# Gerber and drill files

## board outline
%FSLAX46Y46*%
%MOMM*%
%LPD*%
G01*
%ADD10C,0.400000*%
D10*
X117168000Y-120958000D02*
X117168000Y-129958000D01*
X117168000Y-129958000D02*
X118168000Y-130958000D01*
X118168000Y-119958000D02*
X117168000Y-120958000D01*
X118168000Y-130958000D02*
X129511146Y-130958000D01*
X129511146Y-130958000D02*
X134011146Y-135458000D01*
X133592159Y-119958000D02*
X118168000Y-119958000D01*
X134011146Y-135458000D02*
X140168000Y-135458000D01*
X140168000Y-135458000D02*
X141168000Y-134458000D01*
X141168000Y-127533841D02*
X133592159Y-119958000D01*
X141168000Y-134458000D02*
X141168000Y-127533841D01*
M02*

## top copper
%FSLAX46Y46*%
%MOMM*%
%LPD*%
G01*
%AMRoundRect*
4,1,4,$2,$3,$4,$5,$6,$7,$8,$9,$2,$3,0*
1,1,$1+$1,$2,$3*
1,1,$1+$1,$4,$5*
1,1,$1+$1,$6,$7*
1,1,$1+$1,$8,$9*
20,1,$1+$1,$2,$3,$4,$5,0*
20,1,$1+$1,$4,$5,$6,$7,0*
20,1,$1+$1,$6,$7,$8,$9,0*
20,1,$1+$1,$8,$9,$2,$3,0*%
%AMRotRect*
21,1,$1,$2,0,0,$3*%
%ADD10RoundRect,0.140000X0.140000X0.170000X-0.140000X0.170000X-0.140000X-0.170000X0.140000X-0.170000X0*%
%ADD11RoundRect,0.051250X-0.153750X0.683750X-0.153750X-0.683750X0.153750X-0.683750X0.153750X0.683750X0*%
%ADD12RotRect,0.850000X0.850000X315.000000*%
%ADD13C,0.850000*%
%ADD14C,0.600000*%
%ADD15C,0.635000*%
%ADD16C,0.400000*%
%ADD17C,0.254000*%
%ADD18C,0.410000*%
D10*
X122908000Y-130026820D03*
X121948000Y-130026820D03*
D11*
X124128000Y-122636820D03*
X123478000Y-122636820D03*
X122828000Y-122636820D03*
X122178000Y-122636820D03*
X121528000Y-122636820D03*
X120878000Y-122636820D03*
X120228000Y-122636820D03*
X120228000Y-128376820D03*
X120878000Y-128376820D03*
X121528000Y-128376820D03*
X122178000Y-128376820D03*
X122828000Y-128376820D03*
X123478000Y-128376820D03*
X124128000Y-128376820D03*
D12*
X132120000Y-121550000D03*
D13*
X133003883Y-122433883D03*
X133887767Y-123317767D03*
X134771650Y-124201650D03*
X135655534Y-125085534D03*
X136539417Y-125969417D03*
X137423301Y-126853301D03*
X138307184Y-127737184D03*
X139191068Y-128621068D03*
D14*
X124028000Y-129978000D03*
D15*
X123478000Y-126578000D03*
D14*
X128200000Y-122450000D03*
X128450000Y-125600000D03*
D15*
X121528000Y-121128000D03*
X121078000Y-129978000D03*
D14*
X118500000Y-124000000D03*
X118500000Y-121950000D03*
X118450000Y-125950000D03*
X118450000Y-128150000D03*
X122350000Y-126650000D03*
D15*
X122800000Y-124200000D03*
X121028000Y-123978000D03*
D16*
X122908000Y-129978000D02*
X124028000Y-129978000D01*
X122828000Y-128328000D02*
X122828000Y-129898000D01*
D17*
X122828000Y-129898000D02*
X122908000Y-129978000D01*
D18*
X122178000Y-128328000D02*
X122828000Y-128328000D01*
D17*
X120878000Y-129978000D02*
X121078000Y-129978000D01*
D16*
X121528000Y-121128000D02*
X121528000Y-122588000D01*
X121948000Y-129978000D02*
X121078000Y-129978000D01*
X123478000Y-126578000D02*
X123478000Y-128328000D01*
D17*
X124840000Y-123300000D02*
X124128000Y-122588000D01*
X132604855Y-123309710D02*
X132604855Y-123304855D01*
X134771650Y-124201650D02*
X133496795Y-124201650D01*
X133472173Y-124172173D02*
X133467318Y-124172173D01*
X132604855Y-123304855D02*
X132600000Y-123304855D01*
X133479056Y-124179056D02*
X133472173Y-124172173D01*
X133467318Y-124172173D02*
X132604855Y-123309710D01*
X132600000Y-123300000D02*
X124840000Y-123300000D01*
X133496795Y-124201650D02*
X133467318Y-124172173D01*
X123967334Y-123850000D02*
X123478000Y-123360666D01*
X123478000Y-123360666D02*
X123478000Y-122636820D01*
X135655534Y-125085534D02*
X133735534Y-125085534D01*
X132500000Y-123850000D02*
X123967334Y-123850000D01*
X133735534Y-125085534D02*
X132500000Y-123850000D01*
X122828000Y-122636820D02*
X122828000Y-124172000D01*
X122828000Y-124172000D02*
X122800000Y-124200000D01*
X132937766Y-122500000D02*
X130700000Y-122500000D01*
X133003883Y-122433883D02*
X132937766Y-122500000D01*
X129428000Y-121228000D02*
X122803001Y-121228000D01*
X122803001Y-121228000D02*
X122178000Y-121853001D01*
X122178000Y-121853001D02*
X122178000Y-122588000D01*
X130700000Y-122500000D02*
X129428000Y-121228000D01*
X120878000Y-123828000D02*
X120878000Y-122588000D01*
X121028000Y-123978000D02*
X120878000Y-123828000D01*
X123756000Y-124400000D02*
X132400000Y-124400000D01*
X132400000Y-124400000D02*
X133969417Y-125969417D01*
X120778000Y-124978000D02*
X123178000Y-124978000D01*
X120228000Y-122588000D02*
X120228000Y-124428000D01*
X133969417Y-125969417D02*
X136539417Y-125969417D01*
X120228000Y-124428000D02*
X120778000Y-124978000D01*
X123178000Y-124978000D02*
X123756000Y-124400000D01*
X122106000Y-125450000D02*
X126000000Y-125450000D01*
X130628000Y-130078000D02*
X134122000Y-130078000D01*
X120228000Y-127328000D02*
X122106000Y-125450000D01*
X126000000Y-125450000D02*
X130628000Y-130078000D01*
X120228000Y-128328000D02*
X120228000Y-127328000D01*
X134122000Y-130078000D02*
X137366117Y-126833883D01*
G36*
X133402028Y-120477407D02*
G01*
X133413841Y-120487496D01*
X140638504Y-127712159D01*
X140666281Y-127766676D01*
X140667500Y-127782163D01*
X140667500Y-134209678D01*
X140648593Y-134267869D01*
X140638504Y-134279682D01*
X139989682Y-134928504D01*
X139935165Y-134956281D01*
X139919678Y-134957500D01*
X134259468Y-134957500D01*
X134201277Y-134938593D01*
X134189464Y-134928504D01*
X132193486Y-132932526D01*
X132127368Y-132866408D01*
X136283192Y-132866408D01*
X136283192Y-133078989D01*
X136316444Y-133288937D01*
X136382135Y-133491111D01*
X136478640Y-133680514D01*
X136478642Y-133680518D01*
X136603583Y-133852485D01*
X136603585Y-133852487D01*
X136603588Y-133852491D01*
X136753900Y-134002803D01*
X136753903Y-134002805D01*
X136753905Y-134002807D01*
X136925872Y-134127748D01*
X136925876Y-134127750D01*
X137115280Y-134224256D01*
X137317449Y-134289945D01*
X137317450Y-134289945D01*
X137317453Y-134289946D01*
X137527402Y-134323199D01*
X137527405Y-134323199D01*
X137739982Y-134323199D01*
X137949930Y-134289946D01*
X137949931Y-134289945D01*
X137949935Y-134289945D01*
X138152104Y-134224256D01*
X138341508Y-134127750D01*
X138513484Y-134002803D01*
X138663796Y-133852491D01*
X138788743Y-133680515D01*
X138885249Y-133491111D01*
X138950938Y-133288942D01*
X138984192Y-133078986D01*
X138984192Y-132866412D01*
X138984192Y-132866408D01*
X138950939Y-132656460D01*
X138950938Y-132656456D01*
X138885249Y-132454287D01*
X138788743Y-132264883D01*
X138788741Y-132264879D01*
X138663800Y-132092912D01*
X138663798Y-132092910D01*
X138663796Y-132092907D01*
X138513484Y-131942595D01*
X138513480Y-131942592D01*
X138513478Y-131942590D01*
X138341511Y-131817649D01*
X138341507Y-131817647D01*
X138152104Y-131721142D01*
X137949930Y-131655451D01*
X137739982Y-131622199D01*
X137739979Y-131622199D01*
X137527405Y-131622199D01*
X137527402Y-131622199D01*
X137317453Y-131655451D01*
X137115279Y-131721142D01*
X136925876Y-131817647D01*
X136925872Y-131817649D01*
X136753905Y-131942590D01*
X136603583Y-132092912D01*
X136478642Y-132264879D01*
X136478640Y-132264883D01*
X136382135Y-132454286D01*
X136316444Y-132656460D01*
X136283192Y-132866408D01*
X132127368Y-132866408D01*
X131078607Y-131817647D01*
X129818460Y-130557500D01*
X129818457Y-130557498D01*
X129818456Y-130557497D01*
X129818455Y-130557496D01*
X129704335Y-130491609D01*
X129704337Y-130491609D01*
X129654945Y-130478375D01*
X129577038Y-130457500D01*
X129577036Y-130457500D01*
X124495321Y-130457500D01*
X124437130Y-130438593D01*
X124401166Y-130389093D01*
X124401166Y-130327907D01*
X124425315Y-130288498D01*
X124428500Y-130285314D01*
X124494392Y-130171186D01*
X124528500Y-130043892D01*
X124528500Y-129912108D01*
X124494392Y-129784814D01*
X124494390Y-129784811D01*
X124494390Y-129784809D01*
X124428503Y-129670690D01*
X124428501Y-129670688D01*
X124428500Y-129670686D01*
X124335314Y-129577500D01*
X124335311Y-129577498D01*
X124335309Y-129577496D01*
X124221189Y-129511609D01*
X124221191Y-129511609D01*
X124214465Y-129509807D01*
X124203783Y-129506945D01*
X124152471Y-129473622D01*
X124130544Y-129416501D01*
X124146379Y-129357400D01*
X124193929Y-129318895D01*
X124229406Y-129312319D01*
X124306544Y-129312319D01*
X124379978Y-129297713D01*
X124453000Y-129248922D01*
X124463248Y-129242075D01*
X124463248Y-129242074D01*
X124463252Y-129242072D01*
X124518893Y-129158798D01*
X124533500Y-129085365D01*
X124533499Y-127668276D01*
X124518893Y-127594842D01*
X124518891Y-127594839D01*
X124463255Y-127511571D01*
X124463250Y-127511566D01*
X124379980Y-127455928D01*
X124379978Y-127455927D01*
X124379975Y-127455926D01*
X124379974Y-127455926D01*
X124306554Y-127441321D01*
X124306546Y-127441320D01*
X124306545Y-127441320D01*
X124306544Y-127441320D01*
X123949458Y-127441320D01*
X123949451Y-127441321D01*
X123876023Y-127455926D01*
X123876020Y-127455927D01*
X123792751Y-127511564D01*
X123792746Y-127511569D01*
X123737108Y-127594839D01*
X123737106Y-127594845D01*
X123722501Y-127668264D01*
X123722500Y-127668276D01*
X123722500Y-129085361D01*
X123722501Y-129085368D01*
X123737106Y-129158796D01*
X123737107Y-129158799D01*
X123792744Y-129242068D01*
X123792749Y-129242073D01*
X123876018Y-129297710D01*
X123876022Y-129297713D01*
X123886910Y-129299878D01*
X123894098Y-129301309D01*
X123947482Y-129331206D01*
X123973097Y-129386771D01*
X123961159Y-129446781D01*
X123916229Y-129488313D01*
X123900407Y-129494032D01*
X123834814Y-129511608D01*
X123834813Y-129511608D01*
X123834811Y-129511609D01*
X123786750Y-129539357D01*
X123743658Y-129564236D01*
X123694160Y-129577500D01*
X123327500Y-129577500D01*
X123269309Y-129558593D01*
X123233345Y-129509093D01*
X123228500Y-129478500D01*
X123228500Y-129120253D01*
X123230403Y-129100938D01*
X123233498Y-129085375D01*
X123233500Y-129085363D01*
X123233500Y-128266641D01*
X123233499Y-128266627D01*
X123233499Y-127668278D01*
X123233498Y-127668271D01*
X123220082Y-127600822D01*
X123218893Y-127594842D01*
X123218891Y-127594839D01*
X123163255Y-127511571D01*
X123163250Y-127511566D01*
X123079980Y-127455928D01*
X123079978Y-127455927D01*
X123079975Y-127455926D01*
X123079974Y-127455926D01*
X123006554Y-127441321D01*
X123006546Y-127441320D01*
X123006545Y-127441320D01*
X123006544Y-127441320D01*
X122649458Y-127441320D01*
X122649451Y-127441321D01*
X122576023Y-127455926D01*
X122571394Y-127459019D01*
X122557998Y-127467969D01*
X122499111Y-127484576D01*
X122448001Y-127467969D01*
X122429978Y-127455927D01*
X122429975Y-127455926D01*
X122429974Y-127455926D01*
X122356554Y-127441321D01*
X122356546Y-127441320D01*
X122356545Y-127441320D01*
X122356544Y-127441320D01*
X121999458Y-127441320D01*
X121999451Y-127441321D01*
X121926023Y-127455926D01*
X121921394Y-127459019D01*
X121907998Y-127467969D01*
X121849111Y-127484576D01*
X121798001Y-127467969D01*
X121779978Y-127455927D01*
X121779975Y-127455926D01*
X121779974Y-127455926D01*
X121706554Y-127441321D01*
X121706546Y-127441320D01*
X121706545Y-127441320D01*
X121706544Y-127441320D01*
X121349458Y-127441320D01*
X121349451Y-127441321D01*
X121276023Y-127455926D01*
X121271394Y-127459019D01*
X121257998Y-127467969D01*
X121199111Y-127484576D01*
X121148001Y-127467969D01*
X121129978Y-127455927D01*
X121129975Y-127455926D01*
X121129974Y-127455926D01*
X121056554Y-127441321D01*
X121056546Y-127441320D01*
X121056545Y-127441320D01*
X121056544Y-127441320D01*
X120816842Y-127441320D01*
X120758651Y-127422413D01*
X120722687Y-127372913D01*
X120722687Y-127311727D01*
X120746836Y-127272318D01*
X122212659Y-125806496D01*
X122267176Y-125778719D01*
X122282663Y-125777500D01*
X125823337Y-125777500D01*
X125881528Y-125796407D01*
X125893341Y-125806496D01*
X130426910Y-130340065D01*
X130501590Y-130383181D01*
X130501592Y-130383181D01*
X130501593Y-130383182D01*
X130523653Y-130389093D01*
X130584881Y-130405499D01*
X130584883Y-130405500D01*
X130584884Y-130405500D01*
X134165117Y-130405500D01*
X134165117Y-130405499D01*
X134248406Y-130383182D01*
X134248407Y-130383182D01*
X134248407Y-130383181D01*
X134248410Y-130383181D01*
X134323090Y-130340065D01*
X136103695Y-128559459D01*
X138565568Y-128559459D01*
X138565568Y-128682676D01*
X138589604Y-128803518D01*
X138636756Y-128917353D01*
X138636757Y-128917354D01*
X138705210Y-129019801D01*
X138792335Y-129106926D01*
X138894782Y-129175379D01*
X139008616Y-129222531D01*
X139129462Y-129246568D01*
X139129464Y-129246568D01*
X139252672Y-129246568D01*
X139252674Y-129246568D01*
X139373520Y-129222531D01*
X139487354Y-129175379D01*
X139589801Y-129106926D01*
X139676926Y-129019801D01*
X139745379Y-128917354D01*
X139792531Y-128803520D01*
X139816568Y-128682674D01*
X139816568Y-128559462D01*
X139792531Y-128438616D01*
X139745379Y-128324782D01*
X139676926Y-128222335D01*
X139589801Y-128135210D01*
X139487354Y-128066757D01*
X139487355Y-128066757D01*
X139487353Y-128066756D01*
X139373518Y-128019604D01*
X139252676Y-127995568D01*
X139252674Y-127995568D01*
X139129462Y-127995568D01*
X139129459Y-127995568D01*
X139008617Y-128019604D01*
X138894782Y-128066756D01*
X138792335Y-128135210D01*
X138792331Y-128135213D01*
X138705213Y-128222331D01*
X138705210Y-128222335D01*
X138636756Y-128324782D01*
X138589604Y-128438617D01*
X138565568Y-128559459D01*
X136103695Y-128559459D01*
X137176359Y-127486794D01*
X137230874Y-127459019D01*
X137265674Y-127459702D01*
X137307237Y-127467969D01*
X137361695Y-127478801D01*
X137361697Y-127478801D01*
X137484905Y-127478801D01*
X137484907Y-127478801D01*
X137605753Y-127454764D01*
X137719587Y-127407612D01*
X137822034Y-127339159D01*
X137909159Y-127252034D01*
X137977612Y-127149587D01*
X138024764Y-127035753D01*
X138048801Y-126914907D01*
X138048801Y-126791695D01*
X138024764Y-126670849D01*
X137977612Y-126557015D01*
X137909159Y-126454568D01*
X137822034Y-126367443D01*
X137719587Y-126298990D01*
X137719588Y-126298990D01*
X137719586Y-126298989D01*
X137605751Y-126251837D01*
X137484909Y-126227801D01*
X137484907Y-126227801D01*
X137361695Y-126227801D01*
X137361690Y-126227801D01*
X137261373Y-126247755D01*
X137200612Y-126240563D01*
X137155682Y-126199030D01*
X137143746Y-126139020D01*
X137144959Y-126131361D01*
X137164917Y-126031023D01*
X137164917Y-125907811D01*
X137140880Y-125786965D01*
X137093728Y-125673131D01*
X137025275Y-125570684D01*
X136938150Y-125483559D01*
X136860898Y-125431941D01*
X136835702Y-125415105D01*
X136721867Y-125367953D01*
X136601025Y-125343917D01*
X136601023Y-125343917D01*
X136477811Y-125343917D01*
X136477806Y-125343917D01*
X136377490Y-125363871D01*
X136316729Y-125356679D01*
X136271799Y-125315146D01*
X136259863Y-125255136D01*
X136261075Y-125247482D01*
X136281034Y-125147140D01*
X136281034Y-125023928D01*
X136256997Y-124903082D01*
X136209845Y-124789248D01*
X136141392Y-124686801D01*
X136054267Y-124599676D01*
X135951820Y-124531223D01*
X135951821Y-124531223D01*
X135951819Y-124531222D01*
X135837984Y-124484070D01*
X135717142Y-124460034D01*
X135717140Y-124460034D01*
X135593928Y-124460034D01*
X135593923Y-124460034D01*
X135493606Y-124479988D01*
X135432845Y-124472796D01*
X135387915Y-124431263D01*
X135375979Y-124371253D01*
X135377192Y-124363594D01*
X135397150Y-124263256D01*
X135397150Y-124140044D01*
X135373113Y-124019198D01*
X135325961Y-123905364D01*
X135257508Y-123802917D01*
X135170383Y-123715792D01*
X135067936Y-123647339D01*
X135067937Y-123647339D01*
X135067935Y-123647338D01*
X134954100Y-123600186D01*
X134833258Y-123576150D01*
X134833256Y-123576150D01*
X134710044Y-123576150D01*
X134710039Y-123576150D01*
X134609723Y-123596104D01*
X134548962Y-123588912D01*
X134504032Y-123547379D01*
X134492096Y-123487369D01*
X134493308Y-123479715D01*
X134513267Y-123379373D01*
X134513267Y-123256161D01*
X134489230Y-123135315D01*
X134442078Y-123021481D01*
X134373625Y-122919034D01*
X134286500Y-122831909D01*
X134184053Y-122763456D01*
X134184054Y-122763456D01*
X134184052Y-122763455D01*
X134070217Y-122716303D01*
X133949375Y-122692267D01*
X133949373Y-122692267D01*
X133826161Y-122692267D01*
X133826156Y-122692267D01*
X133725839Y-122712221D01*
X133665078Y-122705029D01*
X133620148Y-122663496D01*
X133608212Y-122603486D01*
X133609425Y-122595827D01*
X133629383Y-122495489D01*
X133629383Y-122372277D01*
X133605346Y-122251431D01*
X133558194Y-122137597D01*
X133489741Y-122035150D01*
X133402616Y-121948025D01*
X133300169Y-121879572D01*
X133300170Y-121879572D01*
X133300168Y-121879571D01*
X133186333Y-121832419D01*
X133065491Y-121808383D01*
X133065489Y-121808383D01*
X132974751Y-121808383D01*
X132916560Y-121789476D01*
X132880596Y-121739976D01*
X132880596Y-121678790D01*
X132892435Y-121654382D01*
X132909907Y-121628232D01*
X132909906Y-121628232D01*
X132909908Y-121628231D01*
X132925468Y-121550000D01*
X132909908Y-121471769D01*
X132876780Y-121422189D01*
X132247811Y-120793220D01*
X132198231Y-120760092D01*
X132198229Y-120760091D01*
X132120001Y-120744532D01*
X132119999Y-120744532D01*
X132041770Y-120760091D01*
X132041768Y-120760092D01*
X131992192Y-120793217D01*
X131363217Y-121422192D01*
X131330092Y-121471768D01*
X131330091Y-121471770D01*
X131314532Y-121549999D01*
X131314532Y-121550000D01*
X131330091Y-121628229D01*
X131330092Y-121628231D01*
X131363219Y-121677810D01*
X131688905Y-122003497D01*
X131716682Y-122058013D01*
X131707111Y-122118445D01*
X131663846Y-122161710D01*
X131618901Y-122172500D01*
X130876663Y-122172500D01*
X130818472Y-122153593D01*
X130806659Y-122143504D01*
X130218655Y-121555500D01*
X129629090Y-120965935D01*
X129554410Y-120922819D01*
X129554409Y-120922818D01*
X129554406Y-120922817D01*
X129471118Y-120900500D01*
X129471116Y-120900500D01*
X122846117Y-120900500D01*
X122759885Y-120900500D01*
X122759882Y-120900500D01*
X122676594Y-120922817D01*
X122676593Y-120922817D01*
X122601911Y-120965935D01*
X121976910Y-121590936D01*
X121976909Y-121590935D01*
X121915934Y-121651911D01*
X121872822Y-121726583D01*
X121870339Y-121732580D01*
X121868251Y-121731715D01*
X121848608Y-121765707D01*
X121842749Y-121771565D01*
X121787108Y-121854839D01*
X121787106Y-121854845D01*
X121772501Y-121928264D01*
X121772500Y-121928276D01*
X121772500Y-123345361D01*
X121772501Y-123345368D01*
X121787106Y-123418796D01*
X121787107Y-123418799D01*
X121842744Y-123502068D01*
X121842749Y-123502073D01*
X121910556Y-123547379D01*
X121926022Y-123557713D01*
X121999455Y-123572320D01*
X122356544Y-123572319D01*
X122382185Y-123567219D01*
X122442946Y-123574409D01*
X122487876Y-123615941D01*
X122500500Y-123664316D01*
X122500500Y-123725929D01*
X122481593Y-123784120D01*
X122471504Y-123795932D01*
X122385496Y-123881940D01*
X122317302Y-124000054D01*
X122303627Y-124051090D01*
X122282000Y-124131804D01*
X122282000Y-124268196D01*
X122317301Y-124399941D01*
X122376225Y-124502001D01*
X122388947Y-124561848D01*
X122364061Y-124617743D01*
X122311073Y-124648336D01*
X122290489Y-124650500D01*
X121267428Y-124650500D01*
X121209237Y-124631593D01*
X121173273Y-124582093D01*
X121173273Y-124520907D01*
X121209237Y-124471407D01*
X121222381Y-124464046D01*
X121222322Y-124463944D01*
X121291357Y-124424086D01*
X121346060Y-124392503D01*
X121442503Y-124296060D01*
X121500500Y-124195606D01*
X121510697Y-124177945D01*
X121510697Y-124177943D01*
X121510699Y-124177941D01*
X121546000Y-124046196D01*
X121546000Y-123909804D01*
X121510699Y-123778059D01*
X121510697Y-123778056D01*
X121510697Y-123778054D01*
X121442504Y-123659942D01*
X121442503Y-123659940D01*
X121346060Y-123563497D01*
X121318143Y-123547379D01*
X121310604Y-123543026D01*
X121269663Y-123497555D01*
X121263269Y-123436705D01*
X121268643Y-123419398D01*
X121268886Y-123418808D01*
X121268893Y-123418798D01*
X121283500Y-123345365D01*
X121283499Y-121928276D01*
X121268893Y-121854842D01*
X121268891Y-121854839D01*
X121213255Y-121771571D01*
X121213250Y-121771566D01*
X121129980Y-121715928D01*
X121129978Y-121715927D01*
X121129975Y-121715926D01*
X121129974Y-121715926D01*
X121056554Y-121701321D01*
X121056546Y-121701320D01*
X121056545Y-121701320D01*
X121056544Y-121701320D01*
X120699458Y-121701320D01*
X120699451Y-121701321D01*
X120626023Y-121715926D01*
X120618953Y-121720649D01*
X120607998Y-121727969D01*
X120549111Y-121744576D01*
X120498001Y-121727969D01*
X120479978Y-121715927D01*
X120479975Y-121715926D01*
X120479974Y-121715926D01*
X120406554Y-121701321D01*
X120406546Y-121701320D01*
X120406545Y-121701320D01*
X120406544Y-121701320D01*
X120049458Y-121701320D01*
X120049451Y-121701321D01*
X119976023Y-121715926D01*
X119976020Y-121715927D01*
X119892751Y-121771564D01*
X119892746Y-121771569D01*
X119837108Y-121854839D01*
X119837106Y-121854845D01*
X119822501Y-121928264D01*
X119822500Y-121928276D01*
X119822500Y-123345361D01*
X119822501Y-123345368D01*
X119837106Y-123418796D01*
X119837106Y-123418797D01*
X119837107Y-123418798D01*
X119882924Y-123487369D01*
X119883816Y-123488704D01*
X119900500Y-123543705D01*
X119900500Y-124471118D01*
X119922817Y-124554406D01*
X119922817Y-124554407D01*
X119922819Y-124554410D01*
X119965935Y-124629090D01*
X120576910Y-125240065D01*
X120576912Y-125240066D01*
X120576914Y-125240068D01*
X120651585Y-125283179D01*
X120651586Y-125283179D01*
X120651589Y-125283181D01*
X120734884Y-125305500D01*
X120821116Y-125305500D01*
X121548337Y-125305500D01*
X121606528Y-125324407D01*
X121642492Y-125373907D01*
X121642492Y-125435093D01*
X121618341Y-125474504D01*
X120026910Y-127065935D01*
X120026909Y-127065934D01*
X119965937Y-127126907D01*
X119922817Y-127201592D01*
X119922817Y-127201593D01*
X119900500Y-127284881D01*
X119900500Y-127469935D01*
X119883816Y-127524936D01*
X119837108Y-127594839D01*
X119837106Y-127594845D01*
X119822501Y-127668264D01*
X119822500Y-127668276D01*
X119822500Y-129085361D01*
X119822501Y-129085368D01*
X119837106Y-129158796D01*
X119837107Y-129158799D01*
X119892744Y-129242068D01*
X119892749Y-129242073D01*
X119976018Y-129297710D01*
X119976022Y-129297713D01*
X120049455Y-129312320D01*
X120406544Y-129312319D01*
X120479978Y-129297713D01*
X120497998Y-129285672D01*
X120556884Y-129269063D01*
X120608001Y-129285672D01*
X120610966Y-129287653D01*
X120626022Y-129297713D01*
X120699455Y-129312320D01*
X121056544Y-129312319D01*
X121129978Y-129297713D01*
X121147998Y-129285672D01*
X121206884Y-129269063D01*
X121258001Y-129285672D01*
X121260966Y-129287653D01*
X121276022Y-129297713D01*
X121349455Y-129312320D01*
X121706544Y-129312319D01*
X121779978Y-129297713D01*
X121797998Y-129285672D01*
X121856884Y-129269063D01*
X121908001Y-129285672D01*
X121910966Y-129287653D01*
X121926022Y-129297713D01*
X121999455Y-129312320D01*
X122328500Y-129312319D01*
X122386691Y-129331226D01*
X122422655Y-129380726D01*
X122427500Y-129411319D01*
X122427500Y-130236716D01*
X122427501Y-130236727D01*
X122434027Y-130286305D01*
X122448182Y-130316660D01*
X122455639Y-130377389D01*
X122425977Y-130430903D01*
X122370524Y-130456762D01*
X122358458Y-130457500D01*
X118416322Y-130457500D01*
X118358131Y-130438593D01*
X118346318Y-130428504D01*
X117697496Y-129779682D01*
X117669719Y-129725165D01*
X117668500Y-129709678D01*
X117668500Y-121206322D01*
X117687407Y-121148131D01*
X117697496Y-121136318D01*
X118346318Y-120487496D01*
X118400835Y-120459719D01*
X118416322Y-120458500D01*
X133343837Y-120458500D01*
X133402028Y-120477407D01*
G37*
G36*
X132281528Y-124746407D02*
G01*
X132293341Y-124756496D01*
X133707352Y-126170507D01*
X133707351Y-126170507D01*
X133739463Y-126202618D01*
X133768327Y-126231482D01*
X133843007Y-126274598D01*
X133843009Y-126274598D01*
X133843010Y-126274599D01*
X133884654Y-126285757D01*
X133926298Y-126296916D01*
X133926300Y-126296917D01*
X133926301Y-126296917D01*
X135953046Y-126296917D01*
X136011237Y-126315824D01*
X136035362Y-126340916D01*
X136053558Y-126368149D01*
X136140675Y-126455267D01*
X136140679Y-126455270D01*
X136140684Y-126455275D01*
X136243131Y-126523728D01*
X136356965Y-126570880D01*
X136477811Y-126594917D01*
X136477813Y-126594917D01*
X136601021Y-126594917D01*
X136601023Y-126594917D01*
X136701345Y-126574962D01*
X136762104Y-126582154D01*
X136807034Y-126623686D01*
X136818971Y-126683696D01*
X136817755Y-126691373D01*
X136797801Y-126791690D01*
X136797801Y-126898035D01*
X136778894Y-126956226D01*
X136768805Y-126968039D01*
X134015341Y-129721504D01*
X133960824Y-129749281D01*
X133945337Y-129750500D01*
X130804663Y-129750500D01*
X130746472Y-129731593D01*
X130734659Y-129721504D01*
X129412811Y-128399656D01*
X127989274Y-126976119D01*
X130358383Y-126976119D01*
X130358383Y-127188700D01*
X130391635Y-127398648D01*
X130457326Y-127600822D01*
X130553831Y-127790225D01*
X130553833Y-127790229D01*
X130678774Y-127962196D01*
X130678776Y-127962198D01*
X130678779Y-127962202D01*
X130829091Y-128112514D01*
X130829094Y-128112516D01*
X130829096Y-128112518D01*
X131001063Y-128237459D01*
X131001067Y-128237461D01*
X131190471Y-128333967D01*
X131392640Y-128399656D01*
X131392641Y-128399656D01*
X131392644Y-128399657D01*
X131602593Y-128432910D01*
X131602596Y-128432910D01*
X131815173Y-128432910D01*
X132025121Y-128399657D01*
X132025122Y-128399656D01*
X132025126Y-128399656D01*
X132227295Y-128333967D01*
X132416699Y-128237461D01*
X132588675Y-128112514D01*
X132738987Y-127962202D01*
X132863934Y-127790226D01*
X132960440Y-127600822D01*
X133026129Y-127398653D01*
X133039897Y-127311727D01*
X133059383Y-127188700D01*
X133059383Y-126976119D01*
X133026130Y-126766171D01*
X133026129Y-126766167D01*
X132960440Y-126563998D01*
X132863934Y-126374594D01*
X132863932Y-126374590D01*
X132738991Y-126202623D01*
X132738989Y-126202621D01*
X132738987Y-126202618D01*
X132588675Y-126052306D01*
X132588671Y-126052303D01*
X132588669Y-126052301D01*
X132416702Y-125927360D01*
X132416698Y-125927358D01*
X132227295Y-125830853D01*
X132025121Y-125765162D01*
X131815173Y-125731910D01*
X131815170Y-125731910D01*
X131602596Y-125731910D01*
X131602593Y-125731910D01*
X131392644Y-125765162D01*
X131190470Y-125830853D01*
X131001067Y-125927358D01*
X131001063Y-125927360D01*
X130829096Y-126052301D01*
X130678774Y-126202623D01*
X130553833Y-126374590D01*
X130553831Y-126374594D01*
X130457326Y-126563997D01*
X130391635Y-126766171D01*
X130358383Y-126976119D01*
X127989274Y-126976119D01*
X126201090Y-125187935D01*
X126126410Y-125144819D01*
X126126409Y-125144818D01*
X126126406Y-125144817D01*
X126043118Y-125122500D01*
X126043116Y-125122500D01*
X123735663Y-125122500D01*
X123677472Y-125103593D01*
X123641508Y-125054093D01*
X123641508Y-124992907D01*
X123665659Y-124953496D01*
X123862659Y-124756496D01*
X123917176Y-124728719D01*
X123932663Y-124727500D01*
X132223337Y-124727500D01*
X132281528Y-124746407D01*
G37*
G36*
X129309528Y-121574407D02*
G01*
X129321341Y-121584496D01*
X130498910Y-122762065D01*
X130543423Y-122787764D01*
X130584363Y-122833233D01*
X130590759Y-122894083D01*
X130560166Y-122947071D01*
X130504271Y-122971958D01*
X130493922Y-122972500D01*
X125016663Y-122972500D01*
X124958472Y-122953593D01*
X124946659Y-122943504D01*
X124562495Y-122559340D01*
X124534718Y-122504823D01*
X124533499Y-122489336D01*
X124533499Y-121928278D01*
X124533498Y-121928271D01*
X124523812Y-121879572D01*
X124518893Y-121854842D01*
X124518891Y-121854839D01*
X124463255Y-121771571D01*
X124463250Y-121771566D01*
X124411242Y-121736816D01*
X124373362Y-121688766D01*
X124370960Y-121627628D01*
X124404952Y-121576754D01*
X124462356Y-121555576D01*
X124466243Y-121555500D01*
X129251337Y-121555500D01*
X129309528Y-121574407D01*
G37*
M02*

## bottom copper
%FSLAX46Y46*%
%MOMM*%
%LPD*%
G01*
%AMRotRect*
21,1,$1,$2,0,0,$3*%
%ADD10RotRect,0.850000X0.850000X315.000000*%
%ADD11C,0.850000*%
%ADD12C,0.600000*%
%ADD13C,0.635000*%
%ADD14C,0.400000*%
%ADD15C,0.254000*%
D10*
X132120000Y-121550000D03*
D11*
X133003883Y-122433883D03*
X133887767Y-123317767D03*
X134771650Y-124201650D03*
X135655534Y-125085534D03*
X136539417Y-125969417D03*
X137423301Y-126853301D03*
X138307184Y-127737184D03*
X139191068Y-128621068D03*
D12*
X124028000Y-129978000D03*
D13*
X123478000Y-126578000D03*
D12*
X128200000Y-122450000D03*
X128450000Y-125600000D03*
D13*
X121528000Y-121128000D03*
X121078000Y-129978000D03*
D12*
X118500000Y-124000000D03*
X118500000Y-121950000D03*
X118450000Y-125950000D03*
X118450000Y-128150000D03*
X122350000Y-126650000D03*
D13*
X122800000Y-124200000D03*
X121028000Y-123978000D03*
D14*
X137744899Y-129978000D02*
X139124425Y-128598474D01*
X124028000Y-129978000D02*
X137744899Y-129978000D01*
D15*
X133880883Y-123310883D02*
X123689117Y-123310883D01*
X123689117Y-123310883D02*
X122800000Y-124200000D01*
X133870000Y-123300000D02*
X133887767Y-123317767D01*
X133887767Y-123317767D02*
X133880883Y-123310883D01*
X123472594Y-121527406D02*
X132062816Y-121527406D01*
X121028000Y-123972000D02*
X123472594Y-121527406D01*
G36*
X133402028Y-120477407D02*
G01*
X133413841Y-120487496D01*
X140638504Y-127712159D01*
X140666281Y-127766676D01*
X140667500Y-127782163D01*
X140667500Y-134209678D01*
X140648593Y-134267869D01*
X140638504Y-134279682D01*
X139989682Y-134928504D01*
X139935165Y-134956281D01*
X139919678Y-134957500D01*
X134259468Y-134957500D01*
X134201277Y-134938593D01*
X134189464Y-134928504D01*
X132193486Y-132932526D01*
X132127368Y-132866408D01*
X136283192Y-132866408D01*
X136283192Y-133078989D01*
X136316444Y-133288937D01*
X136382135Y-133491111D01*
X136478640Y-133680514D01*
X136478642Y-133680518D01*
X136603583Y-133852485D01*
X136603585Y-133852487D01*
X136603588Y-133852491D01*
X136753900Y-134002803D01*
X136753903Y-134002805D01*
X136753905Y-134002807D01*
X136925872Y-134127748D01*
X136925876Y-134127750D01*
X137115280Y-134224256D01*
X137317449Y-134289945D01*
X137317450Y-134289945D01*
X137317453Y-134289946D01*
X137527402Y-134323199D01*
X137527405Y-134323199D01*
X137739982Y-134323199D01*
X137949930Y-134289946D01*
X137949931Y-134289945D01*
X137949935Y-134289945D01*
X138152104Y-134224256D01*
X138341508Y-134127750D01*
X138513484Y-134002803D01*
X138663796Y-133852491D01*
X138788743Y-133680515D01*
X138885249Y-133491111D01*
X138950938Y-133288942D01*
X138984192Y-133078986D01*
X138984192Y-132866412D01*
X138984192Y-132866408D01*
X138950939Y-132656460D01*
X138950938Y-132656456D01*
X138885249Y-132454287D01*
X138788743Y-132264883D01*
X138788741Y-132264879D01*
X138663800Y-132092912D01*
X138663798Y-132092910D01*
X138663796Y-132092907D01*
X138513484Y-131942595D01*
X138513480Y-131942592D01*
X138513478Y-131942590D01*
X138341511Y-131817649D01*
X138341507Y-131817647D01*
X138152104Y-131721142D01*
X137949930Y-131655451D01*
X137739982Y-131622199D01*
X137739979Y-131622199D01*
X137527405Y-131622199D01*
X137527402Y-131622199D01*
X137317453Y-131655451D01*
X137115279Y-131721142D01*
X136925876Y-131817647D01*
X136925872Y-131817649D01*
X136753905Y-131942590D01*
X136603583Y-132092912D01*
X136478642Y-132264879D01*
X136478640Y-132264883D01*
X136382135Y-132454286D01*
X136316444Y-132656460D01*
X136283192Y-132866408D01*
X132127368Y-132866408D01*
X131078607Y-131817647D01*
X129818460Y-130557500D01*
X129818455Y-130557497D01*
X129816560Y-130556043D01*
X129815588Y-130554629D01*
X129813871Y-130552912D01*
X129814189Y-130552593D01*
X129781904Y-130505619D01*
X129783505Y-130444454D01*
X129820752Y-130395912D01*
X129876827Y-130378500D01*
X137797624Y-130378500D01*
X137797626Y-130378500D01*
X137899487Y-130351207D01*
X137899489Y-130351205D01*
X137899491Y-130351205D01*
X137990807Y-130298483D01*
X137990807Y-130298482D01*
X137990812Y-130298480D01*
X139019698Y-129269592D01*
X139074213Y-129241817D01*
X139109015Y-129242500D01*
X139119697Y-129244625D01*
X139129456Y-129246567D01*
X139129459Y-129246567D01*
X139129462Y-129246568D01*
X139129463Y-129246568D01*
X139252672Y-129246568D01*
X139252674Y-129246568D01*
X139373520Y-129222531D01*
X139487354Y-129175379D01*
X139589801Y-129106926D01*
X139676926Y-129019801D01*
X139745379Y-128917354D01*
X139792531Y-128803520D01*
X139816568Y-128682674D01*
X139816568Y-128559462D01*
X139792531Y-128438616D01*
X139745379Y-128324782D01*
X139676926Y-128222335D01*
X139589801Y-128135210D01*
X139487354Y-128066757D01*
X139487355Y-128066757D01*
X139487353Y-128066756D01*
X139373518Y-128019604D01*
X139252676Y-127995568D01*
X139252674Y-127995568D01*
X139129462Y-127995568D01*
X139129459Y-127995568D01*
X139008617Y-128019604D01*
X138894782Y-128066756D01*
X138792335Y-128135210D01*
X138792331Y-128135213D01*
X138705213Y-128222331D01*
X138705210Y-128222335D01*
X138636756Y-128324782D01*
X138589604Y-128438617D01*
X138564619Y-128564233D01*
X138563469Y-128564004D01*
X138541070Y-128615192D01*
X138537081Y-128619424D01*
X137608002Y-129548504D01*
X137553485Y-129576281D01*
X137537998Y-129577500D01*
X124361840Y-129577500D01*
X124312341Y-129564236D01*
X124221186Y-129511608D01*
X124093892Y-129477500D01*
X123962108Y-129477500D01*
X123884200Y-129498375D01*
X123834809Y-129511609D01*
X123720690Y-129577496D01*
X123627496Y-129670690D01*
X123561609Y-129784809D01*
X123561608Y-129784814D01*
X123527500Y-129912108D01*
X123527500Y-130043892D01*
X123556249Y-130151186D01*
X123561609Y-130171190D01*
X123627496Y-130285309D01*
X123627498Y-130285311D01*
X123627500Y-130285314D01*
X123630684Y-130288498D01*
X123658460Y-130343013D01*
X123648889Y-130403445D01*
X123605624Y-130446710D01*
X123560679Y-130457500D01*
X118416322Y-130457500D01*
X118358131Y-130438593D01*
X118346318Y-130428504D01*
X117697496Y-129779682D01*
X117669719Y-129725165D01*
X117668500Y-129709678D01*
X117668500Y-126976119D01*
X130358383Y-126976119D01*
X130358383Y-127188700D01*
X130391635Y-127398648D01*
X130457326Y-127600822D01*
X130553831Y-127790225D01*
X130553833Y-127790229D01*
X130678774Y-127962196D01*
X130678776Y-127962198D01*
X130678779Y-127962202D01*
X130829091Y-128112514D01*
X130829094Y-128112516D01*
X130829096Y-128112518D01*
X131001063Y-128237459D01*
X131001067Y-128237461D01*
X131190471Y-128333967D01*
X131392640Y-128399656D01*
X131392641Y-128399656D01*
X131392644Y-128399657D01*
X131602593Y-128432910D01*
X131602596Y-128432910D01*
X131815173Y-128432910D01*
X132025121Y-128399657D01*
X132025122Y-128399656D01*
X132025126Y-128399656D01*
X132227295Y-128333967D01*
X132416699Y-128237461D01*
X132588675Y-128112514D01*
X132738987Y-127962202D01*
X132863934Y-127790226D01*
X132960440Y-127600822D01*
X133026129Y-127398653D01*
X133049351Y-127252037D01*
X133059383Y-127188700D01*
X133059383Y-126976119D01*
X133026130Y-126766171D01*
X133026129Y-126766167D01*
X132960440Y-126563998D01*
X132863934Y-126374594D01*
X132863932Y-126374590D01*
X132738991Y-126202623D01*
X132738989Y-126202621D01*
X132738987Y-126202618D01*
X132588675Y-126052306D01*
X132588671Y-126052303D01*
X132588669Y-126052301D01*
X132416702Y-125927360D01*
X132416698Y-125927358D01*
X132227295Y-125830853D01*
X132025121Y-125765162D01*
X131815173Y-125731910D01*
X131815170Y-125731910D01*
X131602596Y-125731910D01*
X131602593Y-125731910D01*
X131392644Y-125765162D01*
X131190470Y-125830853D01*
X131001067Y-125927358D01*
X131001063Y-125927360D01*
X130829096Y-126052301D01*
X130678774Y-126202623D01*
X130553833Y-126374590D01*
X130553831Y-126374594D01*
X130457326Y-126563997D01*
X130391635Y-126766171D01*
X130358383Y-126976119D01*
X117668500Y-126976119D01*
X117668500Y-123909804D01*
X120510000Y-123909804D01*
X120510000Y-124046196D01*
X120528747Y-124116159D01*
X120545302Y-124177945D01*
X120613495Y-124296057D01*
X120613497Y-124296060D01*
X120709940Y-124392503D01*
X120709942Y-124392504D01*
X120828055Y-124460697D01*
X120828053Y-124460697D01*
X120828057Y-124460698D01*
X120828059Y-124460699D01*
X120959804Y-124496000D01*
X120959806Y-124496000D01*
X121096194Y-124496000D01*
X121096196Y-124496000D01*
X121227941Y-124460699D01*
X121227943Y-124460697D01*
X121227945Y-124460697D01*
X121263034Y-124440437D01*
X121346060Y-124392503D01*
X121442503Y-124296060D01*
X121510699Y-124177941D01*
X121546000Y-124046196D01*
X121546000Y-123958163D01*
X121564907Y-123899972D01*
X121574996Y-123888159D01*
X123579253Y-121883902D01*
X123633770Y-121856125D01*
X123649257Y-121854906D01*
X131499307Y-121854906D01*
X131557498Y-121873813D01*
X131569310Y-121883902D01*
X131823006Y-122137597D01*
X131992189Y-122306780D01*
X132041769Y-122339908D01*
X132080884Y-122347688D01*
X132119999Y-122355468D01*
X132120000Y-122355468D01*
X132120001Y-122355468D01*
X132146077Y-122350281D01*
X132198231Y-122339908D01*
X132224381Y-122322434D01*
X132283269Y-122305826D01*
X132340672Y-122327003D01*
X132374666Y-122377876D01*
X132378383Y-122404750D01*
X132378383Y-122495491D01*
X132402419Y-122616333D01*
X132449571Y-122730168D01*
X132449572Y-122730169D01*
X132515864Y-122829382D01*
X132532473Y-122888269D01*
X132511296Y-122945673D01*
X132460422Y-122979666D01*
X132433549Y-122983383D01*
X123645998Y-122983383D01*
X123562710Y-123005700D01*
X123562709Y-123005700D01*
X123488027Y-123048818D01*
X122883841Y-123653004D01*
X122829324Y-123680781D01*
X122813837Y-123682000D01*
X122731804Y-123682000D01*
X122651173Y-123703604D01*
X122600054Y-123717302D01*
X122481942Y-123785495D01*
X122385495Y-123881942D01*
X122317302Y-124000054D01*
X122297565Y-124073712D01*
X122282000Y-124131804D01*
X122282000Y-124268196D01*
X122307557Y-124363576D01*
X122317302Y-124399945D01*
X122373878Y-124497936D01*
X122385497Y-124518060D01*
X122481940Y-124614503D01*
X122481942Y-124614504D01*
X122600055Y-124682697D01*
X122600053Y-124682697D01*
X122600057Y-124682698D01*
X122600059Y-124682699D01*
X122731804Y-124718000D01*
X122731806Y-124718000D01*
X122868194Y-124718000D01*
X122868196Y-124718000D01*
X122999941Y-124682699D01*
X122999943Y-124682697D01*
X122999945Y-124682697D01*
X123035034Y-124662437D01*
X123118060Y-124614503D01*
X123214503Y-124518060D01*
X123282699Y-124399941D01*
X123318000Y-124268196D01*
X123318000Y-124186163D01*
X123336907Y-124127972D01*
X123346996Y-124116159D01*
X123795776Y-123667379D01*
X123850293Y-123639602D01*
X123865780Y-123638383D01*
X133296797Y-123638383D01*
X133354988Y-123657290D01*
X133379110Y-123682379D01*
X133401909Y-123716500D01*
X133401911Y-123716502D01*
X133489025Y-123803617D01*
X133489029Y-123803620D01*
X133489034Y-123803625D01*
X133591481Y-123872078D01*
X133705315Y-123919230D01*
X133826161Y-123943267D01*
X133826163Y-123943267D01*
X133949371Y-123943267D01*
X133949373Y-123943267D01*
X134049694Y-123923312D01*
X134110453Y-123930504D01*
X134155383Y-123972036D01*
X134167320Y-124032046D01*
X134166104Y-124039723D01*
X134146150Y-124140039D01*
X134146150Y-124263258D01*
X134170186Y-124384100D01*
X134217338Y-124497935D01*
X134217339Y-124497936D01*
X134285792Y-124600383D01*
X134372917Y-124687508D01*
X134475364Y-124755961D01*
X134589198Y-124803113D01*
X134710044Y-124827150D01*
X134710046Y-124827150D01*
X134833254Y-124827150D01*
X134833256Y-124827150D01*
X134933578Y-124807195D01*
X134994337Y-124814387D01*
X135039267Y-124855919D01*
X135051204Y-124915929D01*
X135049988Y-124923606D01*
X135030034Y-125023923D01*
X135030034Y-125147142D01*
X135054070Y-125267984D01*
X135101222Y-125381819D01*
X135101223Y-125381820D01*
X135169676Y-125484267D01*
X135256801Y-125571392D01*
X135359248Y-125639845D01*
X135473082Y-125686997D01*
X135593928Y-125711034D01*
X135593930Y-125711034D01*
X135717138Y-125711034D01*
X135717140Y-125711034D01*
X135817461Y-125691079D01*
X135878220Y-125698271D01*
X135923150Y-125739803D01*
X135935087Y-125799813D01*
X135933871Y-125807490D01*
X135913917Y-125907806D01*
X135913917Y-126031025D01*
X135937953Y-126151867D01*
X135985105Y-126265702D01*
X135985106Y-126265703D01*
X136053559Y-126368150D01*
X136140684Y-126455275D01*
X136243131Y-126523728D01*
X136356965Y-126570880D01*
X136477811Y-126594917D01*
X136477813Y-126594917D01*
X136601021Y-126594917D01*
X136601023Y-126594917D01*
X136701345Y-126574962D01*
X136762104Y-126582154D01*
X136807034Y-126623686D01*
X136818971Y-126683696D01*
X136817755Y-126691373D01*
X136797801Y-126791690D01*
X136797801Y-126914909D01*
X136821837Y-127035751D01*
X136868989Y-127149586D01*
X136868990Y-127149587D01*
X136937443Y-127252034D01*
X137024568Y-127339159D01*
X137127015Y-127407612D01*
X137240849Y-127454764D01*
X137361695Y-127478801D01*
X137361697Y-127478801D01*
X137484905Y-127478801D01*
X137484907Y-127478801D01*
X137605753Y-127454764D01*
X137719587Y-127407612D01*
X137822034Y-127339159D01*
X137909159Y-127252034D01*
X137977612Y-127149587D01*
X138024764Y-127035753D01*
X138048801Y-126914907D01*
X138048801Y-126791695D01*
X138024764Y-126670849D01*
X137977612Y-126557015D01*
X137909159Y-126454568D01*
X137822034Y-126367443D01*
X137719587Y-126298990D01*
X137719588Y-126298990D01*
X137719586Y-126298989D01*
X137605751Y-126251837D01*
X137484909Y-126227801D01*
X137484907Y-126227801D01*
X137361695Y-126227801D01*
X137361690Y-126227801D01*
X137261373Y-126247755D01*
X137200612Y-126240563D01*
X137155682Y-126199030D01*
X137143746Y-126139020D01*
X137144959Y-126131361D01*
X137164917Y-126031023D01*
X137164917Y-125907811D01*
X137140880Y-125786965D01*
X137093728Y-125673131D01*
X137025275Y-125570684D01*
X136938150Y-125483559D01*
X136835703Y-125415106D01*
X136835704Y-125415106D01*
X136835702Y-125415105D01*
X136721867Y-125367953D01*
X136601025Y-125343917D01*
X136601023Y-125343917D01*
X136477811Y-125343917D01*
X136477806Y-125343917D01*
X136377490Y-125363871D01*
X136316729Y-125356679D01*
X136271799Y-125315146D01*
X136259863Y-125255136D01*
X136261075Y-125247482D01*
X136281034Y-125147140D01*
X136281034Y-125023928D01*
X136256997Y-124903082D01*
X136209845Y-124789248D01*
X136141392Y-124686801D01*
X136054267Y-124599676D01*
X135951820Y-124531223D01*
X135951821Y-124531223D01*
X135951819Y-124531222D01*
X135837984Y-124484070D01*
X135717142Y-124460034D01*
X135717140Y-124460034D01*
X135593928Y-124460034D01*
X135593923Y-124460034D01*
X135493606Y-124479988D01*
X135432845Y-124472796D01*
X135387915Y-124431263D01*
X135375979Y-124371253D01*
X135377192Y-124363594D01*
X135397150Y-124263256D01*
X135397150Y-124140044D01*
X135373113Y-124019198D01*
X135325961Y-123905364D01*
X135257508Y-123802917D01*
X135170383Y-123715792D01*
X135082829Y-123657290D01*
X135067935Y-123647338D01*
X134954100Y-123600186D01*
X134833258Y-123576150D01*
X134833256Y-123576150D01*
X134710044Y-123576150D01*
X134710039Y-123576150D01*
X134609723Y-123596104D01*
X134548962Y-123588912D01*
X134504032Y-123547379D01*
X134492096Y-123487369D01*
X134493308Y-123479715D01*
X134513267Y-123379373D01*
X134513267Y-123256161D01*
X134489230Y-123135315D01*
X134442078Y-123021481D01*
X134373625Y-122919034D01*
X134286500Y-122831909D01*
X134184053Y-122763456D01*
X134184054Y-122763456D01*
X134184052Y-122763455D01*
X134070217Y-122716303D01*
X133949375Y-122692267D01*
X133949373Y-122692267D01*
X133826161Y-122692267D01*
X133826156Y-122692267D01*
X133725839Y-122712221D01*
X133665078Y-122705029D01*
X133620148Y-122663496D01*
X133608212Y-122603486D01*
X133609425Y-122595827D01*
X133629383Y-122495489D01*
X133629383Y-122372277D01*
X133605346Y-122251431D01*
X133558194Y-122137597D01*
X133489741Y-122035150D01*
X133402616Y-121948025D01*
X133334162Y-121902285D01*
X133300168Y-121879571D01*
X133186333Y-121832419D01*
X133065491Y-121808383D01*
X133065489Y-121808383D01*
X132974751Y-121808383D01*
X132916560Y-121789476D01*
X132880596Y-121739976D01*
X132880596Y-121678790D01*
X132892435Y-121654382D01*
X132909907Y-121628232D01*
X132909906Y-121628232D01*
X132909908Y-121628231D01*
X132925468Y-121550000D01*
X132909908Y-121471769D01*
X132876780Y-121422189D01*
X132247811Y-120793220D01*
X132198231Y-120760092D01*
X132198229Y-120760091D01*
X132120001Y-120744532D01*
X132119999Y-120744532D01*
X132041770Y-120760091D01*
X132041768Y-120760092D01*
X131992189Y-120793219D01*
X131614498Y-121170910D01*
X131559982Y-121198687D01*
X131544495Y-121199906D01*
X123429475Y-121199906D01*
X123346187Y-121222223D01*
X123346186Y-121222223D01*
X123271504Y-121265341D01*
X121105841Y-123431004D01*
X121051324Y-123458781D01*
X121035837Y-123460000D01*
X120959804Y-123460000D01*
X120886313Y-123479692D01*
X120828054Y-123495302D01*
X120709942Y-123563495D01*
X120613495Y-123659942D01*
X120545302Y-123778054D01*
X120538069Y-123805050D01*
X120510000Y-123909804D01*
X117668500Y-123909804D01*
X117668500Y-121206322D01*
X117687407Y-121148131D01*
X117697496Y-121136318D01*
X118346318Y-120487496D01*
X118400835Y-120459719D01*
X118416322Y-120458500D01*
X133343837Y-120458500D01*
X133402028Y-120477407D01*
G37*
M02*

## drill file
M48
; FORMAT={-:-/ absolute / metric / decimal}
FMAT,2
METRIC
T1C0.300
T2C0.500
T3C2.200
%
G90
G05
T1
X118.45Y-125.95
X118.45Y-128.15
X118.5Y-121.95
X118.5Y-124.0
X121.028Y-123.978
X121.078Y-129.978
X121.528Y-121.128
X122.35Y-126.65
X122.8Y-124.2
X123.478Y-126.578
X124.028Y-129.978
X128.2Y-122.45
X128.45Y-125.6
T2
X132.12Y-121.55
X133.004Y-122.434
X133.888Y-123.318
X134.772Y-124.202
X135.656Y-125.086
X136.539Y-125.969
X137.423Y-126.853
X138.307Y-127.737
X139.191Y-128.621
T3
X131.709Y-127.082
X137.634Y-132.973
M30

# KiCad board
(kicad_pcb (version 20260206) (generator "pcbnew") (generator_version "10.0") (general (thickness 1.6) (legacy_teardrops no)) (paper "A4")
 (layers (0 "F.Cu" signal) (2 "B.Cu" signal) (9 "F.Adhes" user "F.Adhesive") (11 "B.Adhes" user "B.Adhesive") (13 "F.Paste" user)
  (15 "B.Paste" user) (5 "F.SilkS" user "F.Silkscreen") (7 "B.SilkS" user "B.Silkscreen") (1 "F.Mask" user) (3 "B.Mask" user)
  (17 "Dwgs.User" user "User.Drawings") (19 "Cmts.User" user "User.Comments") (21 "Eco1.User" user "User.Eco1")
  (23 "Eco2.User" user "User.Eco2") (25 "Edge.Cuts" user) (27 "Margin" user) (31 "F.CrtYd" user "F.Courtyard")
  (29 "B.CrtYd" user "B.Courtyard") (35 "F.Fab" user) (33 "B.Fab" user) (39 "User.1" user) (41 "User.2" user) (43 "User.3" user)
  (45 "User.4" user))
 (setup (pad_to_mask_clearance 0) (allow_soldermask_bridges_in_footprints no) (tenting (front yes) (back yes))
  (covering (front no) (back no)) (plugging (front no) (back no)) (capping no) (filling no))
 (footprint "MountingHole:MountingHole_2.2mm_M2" (layer "F.Cu") (at 137.633692 132.972699)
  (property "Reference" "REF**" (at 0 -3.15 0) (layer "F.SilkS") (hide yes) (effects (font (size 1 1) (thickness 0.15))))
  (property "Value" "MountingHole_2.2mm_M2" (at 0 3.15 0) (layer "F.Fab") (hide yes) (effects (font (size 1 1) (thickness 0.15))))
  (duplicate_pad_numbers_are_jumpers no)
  (pad "" np_thru_hole circle (at 0 0) (size 2.2 2.2) (drill 2.2) (layers "*.Cu" "*.Mask")))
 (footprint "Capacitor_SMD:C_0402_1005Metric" (layer "F.Cu") (at 122.428 130.02682 180)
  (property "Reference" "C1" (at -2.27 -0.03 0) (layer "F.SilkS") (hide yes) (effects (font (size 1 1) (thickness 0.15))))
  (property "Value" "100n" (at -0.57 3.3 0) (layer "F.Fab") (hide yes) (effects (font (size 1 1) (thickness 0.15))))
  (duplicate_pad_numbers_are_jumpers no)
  (pad "1" smd roundrect (at -0.48 0 180) (size 0.56 0.62) (layers "F.Cu" "F.Mask" "F.Paste") (roundrect_rratio 0.25) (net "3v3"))
  (pad "2" smd roundrect (at 0.48 0 180) (size 0.56 0.62) (layers "F.Cu" "F.Mask" "F.Paste") (roundrect_rratio 0.25) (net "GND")))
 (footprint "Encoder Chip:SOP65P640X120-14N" (layer "F.Cu") (at 122.178 125.50682 -90)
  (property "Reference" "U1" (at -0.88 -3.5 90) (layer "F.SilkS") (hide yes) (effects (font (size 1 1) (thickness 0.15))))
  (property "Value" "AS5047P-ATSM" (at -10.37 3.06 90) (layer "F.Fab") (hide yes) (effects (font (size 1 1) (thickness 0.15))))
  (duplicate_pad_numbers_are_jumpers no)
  (pad "1" smd roundrect (at -2.87 -1.95 270) (size 1.47 0.41) (layers "F.Cu" "F.Mask" "F.Paste") (roundrect_rratio 0.125) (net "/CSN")
   (solder_mask_margin 0.102))
  (pad "2" smd roundrect (at -2.87 -1.3 270) (size 1.47 0.41) (layers "F.Cu" "F.Mask" "F.Paste") (roundrect_rratio 0.125) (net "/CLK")
   (solder_mask_margin 0.102))
  (pad "3" smd roundrect (at -2.87 -0.65 270) (size 1.47 0.41) (layers "F.Cu" "F.Mask" "F.Paste") (roundrect_rratio 0.125) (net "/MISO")
   (solder_mask_margin 0.102))
  (pad "4" smd roundrect (at -2.87 0 270) (size 1.47 0.41) (layers "F.Cu" "F.Mask" "F.Paste") (roundrect_rratio 0.125) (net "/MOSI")
   (solder_mask_margin 0.102))
  (pad "5" smd roundrect (at -2.87 0.65 270) (size 1.47 0.41) (layers "F.Cu" "F.Mask" "F.Paste") (roundrect_rratio 0.125) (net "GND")
   (solder_mask_margin 0.102))
  (pad "6" smd roundrect (at -2.87 1.3 270) (size 1.47 0.41) (layers "F.Cu" "F.Mask" "F.Paste") (roundrect_rratio 0.125) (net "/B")
   (solder_mask_margin 0.102))
  (pad "7" smd roundrect (at -2.87 1.95 270) (size 1.47 0.41) (layers "F.Cu" "F.Mask" "F.Paste") (roundrect_rratio 0.125) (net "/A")
   (solder_mask_margin 0.102))
  (pad "8" smd roundrect (at 2.87 1.95 270) (size 1.47 0.41) (layers "F.Cu" "F.Mask" "F.Paste") (roundrect_rratio 0.125)
   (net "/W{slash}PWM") (solder_mask_margin 0.102))
  (pad "9" smd roundrect (at 2.87 1.3 270) (size 1.47 0.41) (layers "F.Cu" "F.Mask" "F.Paste") (roundrect_rratio 0.125)
   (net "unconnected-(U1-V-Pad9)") (solder_mask_margin 0.102))
  (pad "10" smd roundrect (at 2.87 0.65 270) (size 1.47 0.41) (layers "F.Cu" "F.Mask" "F.Paste") (roundrect_rratio 0.125)
   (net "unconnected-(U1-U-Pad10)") (solder_mask_margin 0.102))
  (pad "11" smd roundrect (at 2.87 0 270) (size 1.47 0.41) (layers "F.Cu" "F.Mask" "F.Paste") (roundrect_rratio 0.125) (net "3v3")
   (solder_mask_margin 0.102))
  (pad "12" smd roundrect (at 2.87 -0.65 270) (size 1.47 0.41) (layers "F.Cu" "F.Mask" "F.Paste") (roundrect_rratio 0.125) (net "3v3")
   (solder_mask_margin 0.102))
  (pad "13" smd roundrect (at 2.87 -1.3 270) (size 1.47 0.41) (layers "F.Cu" "F.Mask" "F.Paste") (roundrect_rratio 0.125) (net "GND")
   (solder_mask_margin 0.102))
  (pad "14" smd roundrect (at 2.87 -1.95 270) (size 1.47 0.41) (layers "F.Cu" "F.Mask" "F.Paste") (roundrect_rratio 0.125)
   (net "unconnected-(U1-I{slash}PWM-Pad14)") (solder_mask_margin 0.102)))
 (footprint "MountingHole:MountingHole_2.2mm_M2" (layer "F.Cu") (at 131.708883 127.08241)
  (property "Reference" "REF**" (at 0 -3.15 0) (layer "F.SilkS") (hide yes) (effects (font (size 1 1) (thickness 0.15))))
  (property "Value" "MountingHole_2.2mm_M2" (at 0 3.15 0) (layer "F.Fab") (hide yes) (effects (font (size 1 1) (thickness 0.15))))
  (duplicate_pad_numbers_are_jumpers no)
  (pad "" np_thru_hole circle (at 0 0) (size 2.2 2.2) (drill 2.2) (layers "*.Cu" "*.Mask")))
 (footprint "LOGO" (layer "B.Cu") (at 122.19 123.56 180)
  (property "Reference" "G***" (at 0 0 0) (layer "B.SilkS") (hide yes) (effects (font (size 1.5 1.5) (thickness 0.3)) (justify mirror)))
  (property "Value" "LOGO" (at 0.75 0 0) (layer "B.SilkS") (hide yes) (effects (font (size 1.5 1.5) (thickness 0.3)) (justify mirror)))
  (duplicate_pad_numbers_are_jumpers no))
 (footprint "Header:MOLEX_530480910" (layer "B.Cu") (at 132.12 121.55 -45)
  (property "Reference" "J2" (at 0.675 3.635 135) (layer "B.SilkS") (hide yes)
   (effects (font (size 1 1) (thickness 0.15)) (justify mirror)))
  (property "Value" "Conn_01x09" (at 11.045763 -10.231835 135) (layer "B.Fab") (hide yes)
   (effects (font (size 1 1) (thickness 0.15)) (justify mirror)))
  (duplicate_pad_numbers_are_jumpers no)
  (pad "1" thru_hole rect (at 0 0 315) (size 0.85 0.85) (drill 0.5) (layers "*.Cu") (remove_unused_layers no) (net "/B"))
  (pad "2" thru_hole circle (at 1.249999 0 315) (size 0.85 0.85) (drill 0.5) (layers "*.Cu") (remove_unused_layers no) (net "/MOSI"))
  (pad "3" thru_hole circle (at 2.5 0 315) (size 0.85 0.85) (drill 0.5) (layers "*.Cu") (remove_unused_layers no) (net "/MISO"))
  (pad "4" thru_hole circle (at 3.749999 0 315) (size 0.85 0.85) (drill 0.5) (layers "*.Cu") (remove_unused_layers no) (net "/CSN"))
  (pad "5" thru_hole circle (at 5 0 315) (size 0.85 0.85) (drill 0.5) (layers "*.Cu") (remove_unused_layers no) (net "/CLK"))
  (pad "6" thru_hole circle (at 6.249999 0 315) (size 0.85 0.85) (drill 0.5) (layers "*.Cu") (remove_unused_layers no) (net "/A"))
  (pad "7" thru_hole circle (at 7.5 0 315) (size 0.85 0.85) (drill 0.5) (layers "*.Cu") (remove_unused_layers no) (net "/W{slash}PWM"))
  (pad "8" thru_hole circle (at 8.75 0 315) (size 0.85 0.85) (drill 0.5) (layers "*.Cu") (remove_unused_layers no) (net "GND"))
  (pad "9" thru_hole circle (at 10 0 315) (size 0.85 0.85) (drill 0.5) (layers "*.Cu") (remove_unused_layers no) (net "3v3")))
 (gr_line (start 117.168 120.958) (end 117.168 129.958) (stroke (width 0.4) (type default)) (layer "Edge.Cuts"))
 (gr_line (start 117.168 129.958) (end 118.168 130.958) (stroke (width 0.4) (type default)) (layer "Edge.Cuts"))
 (gr_line (start 118.168 119.958) (end 117.168 120.958) (stroke (width 0.4) (type default)) (layer "Edge.Cuts"))
 (gr_line (start 118.168 130.958) (end 129.511146 130.958) (stroke (width 0.4) (type default)) (layer "Edge.Cuts"))
 (gr_line (start 129.511146 130.958) (end 134.011146 135.458) (stroke (width 0.4) (type default)) (layer "Edge.Cuts"))
 (gr_line (start 133.592159 119.958) (end 118.168 119.958) (stroke (width 0.4) (type default)) (layer "Edge.Cuts"))
 (gr_line (start 134.011146 135.458) (end 140.168 135.458) (stroke (width 0.4) (type default)) (layer "Edge.Cuts"))
 (gr_line (start 140.168 135.458) (end 141.168 134.458) (stroke (width 0.4) (type default)) (layer "Edge.Cuts"))
 (gr_line (start 141.168 127.533841) (end 133.592159 119.958) (stroke (width 0.4) (type default)) (layer "Edge.Cuts"))
 (gr_line (start 141.168 134.458) (end 141.168 127.533841) (stroke (width 0.4) (type default)) (layer "Edge.Cuts"))
 (segment (start 122.908 129.978) (end 124.028 129.978) (width 0.4) (layer "F.Cu") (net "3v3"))
 (segment (start 122.828 128.328) (end 122.828 129.898) (width 0.4) (layer "F.Cu") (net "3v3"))
 (segment (start 122.828 129.898) (end 122.908 129.978) (width 0.254) (layer "F.Cu") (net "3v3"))
 (segment (start 122.178 128.328) (end 122.828 128.328) (width 0.41) (layer "F.Cu") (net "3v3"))
 (via (at 124.028 129.978) (size 0.6) (drill 0.3) (layers "F.Cu" "B.Cu") (capping no) (covering (front no) (back no))
  (plugging (front no) (back no)) (filling no) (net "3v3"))
 (segment (start 137.744899 129.978) (end 139.124425 128.598474) (width 0.4) (layer "B.Cu") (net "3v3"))
 (segment (start 124.028 129.978) (end 137.744899 129.978) (width 0.4) (layer "B.Cu") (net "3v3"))
 (segment (start 120.878 129.978) (end 121.078 129.978) (width 0.254) (layer "F.Cu") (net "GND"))
 (segment (start 121.528 121.128) (end 121.528 122.588) (width 0.4) (layer "F.Cu") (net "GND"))
 (segment (start 121.948 129.978) (end 121.078 129.978) (width 0.4) (layer "F.Cu") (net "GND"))
 (segment (start 123.478 126.578) (end 123.478 128.328) (width 0.4) (layer "F.Cu") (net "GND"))
 (via (at 123.478 126.578) (size 0.635) (drill 0.3) (layers "F.Cu" "B.Cu") (free yes) (capping no) (covering (front no) (back no))
  (plugging (front no) (back no)) (filling no) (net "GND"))
 (via (at 128.2 122.45) (size 0.6) (drill 0.3) (layers "F.Cu" "B.Cu") (free yes) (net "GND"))
 (via (at 128.45 125.6) (size 0.6) (drill 0.3) (layers "F.Cu" "B.Cu") (free yes) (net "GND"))
 (via (at 121.528 121.128) (size 0.635) (drill 0.3) (layers "F.Cu" "B.Cu") (capping no) (covering (front no) (back no))
  (plugging (front no) (back no)) (filling no) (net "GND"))
 (via (at 121.078 129.978) (size 0.635) (drill 0.3) (layers "F.Cu" "B.Cu") (free yes) (capping no) (covering (front no) (back no))
  (plugging (front no) (back no)) (filling no) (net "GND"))
 (via (at 118.5 124) (size 0.6) (drill 0.3) (layers "F.Cu" "B.Cu") (free yes) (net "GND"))
 (via (at 118.5 121.95) (size 0.6) (drill 0.3) (layers "F.Cu" "B.Cu") (free yes) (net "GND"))
 (via (at 118.45 125.95) (size 0.6) (drill 0.3) (layers "F.Cu" "B.Cu") (free yes) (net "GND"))
 (via (at 118.45 128.15) (size 0.6) (drill 0.3) (layers "F.Cu" "B.Cu") (free yes) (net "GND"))
 (via (at 122.35 126.65) (size 0.6) (drill 0.3) (layers "F.Cu" "B.Cu") (free yes) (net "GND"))
 (segment (start 124.84 123.3) (end 124.128 122.588) (width 0.254) (layer "F.Cu") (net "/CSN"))
 (segment (start 132.604855 123.30971) (end 132.604855 123.304855) (width 0.254) (layer "F.Cu") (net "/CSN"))
 (segment (start 134.77165 124.20165) (end 133.496795 124.20165) (width 0.254) (layer "F.Cu") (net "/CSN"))
 (segment (start 133.472173 124.172173) (end 133.467318 124.172173) (width 0.254) (layer "F.Cu") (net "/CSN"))
 (segment (start 132.604855 123.304855) (end 132.6 123.304855) (width 0.254) (layer "F.Cu") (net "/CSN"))
 (segment (start 133.479056 124.179056) (end 133.472173 124.172173) (width 0.254) (layer "F.Cu") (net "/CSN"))
 (segment (start 133.467318 124.172173) (end 132.604855 123.30971) (width 0.254) (layer "F.Cu") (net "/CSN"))
 (segment (start 132.6 123.3) (end 124.84 123.3) (width 0.254) (layer "F.Cu") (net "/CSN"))
 (segment (start 133.496795 124.20165) (end 133.467318 124.172173) (width 0.254) (layer "F.Cu") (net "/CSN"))
 (segment (start 123.967334 123.85) (end 123.478 123.360666) (width 0.254) (layer "F.Cu") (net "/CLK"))
 (segment (start 123.478 123.360666) (end 123.478 122.63682) (width 0.254) (layer "F.Cu") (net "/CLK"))
 (segment (start 135.655534 125.085534) (end 133.735534 125.085534) (width 0.254) (layer "F.Cu") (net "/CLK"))
 (segment (start 132.5 123.85) (end 123.967334 123.85) (width 0.254) (layer "F.Cu") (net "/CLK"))
 (segment (start 133.735534 125.085534) (end 132.5 123.85) (width 0.254) (layer "F.Cu") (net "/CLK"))
 (segment (start 122.828 122.63682) (end 122.828 124.172) (width 0.254) (layer "F.Cu") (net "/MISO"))
 (segment (start 122.828 124.172) (end 122.8 124.2) (width 0.254) (layer "F.Cu") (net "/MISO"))
 (via (at 122.8 124.2) (size 0.635) (drill 0.3) (layers "F.Cu" "B.Cu") (capping no) (covering (front no) (back no))
  (plugging (front no) (back no)) (filling no) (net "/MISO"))
 (segment (start 133.880883 123.310883) (end 123.689117 123.310883) (width 0.254) (layer "B.Cu") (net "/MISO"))
 (segment (start 123.689117 123.310883) (end 122.8 124.2) (width 0.254) (layer "B.Cu") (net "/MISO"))
 (segment (start 133.87 123.3) (end 133.887767 123.317767) (width 0.254) (layer "B.Cu") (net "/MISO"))
 (segment (start 133.887767 123.317767) (end 133.880883 123.310883) (width 0.254) (layer "B.Cu") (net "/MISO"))
 (segment (start 132.937766 122.5) (end 130.7 122.5) (width 0.254) (layer "F.Cu") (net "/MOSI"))
 (segment (start 133.003883 122.433883) (end 132.937766 122.5) (width 0.254) (layer "F.Cu") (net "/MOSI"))
 (segment (start 129.428 121.228) (end 122.803001 121.228) (width 0.254) (layer "F.Cu") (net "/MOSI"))
 (segment (start 122.803001 121.228) (end 122.178 121.853001) (width 0.254) (layer "F.Cu") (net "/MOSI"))
 (segment (start 122.178 121.853001) (end 122.178 122.588) (width 0.254) (layer "F.Cu") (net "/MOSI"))
 (segment (start 130.7 122.5) (end 129.428 121.228) (width 0.254) (layer "F.Cu") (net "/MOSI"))
 (segment (start 120.878 123.828) (end 120.878 122.588) (width 0.254) (layer "F.Cu") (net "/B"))
 (segment (start 121.028 123.978) (end 120.878 123.828) (width 0.254) (layer "F.Cu") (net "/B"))
 (via (at 121.028 123.978) (size 0.635) (drill 0.3) (layers "F.Cu" "B.Cu") (capping no) (covering (front no) (back no))
  (plugging (front no) (back no)) (filling no) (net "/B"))
 (segment (start 123.472594 121.527406) (end 132.062816 121.527406) (width 0.254) (layer "B.Cu") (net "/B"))
 (segment (start 121.028 123.972) (end 123.472594 121.527406) (width 0.254) (layer "B.Cu") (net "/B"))
 (segment (start 123.756 124.4) (end 132.4 124.4) (width 0.254) (layer "F.Cu") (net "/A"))
 (segment (start 132.4 124.4) (end 133.969417 125.969417) (width 0.254) (layer "F.Cu") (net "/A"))
 (segment (start 120.778 124.978) (end 123.178 124.978) (width 0.254) (layer "F.Cu") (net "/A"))
 (segment (start 120.228 122.588) (end 120.228 124.428) (width 0.254) (layer "F.Cu") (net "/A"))
 (segment (start 133.969417 125.969417) (end 136.539417 125.969417) (width 0.254) (layer "F.Cu") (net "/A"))
 (segment (start 120.228 124.428) (end 120.778 124.978) (width 0.254) (layer "F.Cu") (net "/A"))
 (segment (start 123.178 124.978) (end 123.756 124.4) (width 0.254) (layer "F.Cu") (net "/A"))
 (segment (start 122.106 125.45) (end 126 125.45) (width 0.254) (layer "F.Cu") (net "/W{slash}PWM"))
 (segment (start 130.628 130.078) (end 134.122 130.078) (width 0.254) (layer "F.Cu") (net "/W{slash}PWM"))
 (segment (start 120.228 127.328) (end 122.106 125.45) (width 0.254) (layer "F.Cu") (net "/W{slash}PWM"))
 (segment (start 126 125.45) (end 130.628 130.078) (width 0.254) (layer "F.Cu") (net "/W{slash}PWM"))
 (segment (start 120.228 128.328) (end 120.228 127.328) (width 0.254) (layer "F.Cu") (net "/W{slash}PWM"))
 (segment (start 134.122 130.078) (end 137.366117 126.833883) (width 0.254) (layer "F.Cu") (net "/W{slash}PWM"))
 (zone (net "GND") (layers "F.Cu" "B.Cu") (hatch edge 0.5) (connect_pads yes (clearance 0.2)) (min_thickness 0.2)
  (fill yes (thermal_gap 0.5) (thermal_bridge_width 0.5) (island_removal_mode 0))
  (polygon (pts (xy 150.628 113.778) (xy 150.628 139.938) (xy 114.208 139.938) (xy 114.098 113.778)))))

